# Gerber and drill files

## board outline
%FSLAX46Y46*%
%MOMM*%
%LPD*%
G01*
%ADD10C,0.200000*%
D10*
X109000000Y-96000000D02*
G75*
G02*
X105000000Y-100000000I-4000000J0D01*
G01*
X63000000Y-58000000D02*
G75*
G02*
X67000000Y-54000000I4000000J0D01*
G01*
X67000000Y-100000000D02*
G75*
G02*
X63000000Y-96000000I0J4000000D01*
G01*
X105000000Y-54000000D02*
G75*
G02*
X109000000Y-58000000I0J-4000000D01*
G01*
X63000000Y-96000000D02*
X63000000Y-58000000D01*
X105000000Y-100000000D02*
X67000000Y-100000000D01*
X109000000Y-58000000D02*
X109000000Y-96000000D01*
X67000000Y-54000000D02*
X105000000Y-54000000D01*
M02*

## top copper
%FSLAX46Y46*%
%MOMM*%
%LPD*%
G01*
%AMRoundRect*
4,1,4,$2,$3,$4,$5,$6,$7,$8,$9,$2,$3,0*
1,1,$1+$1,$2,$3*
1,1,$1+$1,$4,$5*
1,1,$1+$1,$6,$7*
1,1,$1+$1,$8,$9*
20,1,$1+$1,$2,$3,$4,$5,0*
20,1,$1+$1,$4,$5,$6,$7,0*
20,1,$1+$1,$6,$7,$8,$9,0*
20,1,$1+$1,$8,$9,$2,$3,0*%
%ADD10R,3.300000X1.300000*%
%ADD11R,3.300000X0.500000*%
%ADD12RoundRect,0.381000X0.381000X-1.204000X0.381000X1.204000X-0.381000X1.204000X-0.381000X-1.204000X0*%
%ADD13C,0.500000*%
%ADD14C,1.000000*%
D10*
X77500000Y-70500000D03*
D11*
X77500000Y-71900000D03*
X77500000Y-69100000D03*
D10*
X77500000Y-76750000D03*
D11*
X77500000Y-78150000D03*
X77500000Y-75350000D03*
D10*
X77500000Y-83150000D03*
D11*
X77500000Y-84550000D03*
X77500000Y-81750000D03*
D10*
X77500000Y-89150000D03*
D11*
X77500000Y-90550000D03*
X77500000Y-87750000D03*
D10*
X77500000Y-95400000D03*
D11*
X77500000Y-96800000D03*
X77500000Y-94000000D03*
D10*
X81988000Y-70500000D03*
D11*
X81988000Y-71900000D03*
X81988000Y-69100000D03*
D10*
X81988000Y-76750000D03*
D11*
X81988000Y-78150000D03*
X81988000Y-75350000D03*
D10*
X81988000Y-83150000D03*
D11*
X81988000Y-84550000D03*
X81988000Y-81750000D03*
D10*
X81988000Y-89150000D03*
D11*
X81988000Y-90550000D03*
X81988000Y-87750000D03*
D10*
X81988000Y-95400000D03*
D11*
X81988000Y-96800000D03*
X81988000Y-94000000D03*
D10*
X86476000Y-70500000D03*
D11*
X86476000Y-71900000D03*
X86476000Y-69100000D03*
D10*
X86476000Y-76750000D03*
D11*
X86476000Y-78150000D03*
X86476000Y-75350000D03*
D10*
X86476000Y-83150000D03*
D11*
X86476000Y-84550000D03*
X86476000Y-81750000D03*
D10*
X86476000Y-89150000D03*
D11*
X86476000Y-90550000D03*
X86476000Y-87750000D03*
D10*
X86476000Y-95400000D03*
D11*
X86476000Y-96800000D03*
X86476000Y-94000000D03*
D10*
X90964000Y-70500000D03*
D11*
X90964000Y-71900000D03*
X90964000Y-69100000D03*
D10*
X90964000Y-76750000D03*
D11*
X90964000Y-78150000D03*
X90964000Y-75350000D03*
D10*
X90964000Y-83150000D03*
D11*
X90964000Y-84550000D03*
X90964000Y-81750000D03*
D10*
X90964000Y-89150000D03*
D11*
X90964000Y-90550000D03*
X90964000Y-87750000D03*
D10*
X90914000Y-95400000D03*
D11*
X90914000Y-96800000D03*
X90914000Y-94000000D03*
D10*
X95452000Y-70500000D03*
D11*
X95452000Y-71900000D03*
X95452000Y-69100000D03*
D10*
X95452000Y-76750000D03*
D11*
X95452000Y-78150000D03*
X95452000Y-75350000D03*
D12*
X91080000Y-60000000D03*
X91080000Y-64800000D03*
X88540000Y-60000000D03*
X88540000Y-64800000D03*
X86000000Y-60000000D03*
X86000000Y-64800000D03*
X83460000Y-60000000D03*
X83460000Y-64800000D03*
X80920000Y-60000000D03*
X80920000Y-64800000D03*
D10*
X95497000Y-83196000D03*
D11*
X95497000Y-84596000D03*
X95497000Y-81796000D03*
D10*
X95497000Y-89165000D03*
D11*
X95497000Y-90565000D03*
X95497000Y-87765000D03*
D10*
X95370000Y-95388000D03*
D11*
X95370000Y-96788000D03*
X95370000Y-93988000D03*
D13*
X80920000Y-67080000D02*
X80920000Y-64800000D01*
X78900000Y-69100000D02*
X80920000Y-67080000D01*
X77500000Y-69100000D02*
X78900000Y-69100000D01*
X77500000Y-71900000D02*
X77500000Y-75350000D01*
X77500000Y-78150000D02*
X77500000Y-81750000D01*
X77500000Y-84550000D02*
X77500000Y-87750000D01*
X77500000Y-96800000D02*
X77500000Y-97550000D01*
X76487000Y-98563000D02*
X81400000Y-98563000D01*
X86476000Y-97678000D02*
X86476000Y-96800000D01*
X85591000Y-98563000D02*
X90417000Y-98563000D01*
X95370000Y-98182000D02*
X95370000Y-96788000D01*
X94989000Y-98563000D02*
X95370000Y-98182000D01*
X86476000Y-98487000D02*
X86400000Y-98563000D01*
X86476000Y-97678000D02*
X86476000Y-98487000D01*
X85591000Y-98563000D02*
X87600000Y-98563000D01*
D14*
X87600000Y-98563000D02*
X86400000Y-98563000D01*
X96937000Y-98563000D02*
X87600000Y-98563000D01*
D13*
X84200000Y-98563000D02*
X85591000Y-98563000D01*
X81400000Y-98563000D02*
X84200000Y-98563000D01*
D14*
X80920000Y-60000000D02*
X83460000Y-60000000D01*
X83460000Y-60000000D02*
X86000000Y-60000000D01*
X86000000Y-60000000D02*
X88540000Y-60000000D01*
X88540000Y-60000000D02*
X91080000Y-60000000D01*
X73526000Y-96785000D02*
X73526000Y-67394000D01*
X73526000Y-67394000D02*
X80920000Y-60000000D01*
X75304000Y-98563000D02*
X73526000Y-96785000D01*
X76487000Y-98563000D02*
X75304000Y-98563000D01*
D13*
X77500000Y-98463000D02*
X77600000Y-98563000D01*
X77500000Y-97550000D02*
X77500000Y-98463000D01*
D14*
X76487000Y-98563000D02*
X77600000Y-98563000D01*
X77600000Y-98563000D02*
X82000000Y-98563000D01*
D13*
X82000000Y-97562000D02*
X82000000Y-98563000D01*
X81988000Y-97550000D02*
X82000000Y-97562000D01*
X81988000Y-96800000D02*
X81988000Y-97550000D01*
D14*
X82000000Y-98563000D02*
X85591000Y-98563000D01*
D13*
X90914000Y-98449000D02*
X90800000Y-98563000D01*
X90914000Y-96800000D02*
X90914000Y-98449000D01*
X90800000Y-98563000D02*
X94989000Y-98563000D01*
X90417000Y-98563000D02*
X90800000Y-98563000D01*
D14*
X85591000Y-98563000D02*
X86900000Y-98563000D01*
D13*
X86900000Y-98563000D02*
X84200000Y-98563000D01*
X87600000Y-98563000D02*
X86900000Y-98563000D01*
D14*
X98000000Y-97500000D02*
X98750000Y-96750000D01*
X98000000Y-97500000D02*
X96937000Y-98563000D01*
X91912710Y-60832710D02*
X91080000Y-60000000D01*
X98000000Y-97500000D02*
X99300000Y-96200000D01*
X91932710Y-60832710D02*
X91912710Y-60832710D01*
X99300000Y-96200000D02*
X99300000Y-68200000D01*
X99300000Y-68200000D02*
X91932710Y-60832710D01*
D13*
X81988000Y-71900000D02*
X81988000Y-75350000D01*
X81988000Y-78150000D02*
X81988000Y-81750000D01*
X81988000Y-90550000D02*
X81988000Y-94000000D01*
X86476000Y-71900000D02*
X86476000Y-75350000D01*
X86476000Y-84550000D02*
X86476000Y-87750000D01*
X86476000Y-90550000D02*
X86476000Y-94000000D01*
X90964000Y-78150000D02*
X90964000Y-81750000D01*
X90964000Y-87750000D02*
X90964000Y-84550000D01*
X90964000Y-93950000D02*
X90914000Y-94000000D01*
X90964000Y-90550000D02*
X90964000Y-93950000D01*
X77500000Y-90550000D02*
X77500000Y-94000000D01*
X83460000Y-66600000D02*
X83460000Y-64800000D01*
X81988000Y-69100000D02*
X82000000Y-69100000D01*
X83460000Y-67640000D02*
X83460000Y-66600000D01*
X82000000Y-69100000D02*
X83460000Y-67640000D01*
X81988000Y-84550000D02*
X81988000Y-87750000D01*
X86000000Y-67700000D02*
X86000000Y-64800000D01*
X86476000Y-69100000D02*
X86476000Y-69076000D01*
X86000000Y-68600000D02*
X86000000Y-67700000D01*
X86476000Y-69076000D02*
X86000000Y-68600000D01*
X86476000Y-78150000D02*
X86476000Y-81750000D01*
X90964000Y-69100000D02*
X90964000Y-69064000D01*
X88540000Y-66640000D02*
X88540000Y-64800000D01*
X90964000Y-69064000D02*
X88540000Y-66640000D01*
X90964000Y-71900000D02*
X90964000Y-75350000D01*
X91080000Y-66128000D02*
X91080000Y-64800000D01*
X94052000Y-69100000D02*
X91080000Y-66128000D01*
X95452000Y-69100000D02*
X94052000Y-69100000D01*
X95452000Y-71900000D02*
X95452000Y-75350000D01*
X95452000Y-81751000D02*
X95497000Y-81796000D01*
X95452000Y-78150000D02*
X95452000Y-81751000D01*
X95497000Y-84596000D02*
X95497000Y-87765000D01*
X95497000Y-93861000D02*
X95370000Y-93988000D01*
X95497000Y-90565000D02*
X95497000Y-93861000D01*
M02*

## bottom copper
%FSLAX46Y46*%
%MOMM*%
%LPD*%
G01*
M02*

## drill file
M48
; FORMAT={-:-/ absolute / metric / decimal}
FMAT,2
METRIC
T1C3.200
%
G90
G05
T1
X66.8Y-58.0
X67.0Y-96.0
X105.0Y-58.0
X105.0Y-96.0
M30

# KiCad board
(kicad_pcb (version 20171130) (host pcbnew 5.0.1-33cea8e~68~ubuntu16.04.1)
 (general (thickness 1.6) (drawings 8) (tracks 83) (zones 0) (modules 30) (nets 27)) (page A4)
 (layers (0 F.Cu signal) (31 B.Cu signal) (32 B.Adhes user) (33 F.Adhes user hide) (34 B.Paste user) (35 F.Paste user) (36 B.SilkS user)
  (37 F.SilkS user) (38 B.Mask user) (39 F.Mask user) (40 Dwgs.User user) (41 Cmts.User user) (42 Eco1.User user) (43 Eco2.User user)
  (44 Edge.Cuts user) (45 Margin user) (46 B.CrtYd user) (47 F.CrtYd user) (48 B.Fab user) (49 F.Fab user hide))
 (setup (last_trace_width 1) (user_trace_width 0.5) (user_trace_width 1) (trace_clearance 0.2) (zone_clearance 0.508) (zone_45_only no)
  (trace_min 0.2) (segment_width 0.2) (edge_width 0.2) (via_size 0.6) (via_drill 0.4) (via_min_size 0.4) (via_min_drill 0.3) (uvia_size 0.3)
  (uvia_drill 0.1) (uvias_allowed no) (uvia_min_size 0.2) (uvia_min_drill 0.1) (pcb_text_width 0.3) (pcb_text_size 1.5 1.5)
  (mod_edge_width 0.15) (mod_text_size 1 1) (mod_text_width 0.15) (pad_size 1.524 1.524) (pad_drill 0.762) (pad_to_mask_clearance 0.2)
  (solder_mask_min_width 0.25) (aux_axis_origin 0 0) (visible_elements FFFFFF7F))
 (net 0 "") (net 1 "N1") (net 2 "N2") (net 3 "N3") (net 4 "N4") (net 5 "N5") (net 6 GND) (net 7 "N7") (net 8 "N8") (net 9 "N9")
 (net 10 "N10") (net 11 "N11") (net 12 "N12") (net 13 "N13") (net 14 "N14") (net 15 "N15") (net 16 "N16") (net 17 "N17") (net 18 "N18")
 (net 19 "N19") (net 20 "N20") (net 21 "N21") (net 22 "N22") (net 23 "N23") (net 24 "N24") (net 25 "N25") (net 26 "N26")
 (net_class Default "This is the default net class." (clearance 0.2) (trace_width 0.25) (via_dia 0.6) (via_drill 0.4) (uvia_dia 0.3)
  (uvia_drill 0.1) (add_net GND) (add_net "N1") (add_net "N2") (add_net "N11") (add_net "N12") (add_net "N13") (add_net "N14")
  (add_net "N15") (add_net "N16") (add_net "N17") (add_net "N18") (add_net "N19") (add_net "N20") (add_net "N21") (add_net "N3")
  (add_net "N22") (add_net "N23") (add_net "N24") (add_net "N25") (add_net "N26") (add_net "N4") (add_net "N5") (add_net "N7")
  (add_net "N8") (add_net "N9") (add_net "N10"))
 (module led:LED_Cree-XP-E (layer F.Cu) (at 77.5 70.5 90)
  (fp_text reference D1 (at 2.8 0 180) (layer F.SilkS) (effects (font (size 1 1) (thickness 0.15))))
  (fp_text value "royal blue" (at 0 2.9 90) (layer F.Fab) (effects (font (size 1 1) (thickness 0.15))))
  (pad 3 smd rect (at 0 -1 90) (size 1.01 0.75) (layers F.Paste))
  (pad 3 smd rect (at 0 1 90) (size 1.01 0.75) (layers F.Paste))
  (pad 3 smd rect (at 0 0 90) (size 1.01 0.75) (layers F.Paste))
  (pad 3 smd rect (at 0 0 90) (size 1.3 3.3) (layers F.Cu F.Mask))
  (pad 1 smd rect (at -1.4 0 90) (size 0.5 3.3) (layers F.Cu F.Paste F.Mask) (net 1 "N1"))
  (pad 2 smd rect (at 1.4 0 90) (size 0.5 3.3) (layers F.Cu F.Paste F.Mask) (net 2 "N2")))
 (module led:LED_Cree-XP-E (layer F.Cu) (at 77.5 76.75 90)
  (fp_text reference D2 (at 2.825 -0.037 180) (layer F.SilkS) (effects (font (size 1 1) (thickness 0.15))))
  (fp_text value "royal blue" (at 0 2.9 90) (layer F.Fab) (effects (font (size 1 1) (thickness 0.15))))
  (pad 3 smd rect (at 0 -1 90) (size 1.01 0.75) (layers F.Paste))
  (pad 3 smd rect (at 0 1 90) (size 1.01 0.75) (layers F.Paste))
  (pad 3 smd rect (at 0 0 90) (size 1.01 0.75) (layers F.Paste))
  (pad 3 smd rect (at 0 0 90) (size 1.3 3.3) (layers F.Cu F.Mask))
  (pad 1 smd rect (at -1.4 0 90) (size 0.5 3.3) (layers F.Cu F.Paste F.Mask) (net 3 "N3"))
  (pad 2 smd rect (at 1.4 0 90) (size 0.5 3.3) (layers F.Cu F.Paste F.Mask) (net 1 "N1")))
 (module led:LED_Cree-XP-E (layer F.Cu) (at 77.5 83.15 90)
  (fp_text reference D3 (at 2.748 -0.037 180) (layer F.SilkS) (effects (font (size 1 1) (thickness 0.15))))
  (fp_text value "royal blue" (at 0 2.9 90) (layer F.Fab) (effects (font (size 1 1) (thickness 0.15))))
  (pad 3 smd rect (at 0 -1 90) (size 1.01 0.75) (layers F.Paste))
  (pad 3 smd rect (at 0 1 90) (size 1.01 0.75) (layers F.Paste))
  (pad 3 smd rect (at 0 0 90) (size 1.01 0.75) (layers F.Paste))
  (pad 3 smd rect (at 0 0 90) (size 1.3 3.3) (layers F.Cu F.Mask))
  (pad 1 smd rect (at -1.4 0 90) (size 0.5 3.3) (layers F.Cu F.Paste F.Mask) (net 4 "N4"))
  (pad 2 smd rect (at 1.4 0 90) (size 0.5 3.3) (layers F.Cu F.Paste F.Mask) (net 3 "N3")))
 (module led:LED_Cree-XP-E (layer F.Cu) (at 77.5 89.15 90)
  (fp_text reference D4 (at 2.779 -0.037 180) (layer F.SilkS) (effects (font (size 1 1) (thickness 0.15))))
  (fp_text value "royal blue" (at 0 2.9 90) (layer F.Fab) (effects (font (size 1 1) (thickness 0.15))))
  (pad 3 smd rect (at 0 -1 90) (size 1.01 0.75) (layers F.Paste))
  (pad 3 smd rect (at 0 1 90) (size 1.01 0.75) (layers F.Paste))
  (pad 3 smd rect (at 0 0 90) (size 1.01 0.75) (layers F.Paste))
  (pad 3 smd rect (at 0 0 90) (size 1.3 3.3) (layers F.Cu F.Mask))
  (pad 1 smd rect (at -1.4 0 90) (size 0.5 3.3) (layers F.Cu F.Paste F.Mask) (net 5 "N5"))
  (pad 2 smd rect (at 1.4 0 90) (size 0.5 3.3) (layers F.Cu F.Paste F.Mask) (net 4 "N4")))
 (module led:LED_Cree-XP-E (layer F.Cu) (at 77.5 95.4 90)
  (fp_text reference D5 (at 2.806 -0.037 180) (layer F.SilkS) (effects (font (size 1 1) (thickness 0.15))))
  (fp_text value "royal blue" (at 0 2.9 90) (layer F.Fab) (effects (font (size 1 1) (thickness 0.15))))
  (pad 3 smd rect (at 0 -1 90) (size 1.01 0.75) (layers F.Paste))
  (pad 3 smd rect (at 0 1 90) (size 1.01 0.75) (layers F.Paste))
  (pad 3 smd rect (at 0 0 90) (size 1.01 0.75) (layers F.Paste))
  (pad 3 smd rect (at 0 0 90) (size 1.3 3.3) (layers F.Cu F.Mask))
  (pad 1 smd rect (at -1.4 0 90) (size 0.5 3.3) (layers F.Cu F.Paste F.Mask) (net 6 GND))
  (pad 2 smd rect (at 1.4 0 90) (size 0.5 3.3) (layers F.Cu F.Paste F.Mask) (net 5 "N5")))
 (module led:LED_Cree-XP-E (layer F.Cu) (at 81.988 70.5 90)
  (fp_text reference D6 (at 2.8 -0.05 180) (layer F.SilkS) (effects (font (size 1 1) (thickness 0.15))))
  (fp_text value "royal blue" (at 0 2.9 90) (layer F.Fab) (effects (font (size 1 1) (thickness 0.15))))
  (pad 3 smd rect (at 0 -1 90) (size 1.01 0.75) (layers F.Paste))
  (pad 3 smd rect (at 0 1 90) (size 1.01 0.75) (layers F.Paste))
  (pad 3 smd rect (at 0 0 90) (size 1.01 0.75) (layers F.Paste))
  (pad 3 smd rect (at 0 0 90) (size 1.3 3.3) (layers F.Cu F.Mask))
  (pad 1 smd rect (at -1.4 0 90) (size 0.5 3.3) (layers F.Cu F.Paste F.Mask) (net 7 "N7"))
  (pad 2 smd rect (at 1.4 0 90) (size 0.5 3.3) (layers F.Cu F.Paste F.Mask) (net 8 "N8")))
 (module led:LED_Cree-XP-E (layer F.Cu) (at 81.988 76.75 90)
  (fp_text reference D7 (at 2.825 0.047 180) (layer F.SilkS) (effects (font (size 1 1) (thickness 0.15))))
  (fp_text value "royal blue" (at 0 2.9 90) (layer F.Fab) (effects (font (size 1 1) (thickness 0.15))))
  (pad 3 smd rect (at 0 -1 90) (size 1.01 0.75) (layers F.Paste))
  (pad 3 smd rect (at 0 1 90) (size 1.01 0.75) (layers F.Paste))
  (pad 3 smd rect (at 0 0 90) (size 1.01 0.75) (layers F.Paste))
  (pad 3 smd rect (at 0 0 90) (size 1.3 3.3) (layers F.Cu F.Mask))
  (pad 1 smd rect (at -1.4 0 90) (size 0.5 3.3) (layers F.Cu F.Paste F.Mask) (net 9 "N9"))
  (pad 2 smd rect (at 1.4 0 90) (size 0.5 3.3) (layers F.Cu F.Paste F.Mask) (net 7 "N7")))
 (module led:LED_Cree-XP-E (layer F.Cu) (at 81.988 83.15 90)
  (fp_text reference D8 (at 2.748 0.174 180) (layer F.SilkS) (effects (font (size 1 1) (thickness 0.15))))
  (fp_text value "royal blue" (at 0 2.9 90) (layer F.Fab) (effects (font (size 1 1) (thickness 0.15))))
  (pad 3 smd rect (at 0 -1 90) (size 1.01 0.75) (layers F.Paste))
  (pad 3 smd rect (at 0 1 90) (size 1.01 0.75) (layers F.Paste))
  (pad 3 smd rect (at 0 0 90) (size 1.01 0.75) (layers F.Paste))
  (pad 3 smd rect (at 0 0 90) (size 1.3 3.3) (layers F.Cu F.Mask))
  (pad 1 smd rect (at -1.4 0 90) (size 0.5 3.3) (layers F.Cu F.Paste F.Mask) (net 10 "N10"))
  (pad 2 smd rect (at 1.4 0 90) (size 0.5 3.3) (layers F.Cu F.Paste F.Mask) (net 9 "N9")))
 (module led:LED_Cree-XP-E (layer F.Cu) (at 81.988 89.15 90)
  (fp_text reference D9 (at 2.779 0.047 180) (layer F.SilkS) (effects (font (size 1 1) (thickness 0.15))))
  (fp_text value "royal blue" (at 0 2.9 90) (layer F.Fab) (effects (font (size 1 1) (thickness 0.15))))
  (pad 3 smd rect (at 0 -1 90) (size 1.01 0.75) (layers F.Paste))
  (pad 3 smd rect (at 0 1 90) (size 1.01 0.75) (layers F.Paste))
  (pad 3 smd rect (at 0 0 90) (size 1.01 0.75) (layers F.Paste))
  (pad 3 smd rect (at 0 0 90) (size 1.3 3.3) (layers F.Cu F.Mask))
  (pad 1 smd rect (at -1.4 0 90) (size 0.5 3.3) (layers F.Cu F.Paste F.Mask) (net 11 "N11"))
  (pad 2 smd rect (at 1.4 0 90) (size 0.5 3.3) (layers F.Cu F.Paste F.Mask) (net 10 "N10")))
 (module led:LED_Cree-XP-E (layer F.Cu) (at 81.988 95.4 90)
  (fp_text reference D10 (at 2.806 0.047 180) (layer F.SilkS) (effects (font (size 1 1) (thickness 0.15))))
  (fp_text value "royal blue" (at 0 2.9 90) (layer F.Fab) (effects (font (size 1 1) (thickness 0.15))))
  (pad 3 smd rect (at 0 -1 90) (size 1.01 0.75) (layers F.Paste))
  (pad 3 smd rect (at 0 1 90) (size 1.01 0.75) (layers F.Paste))
  (pad 3 smd rect (at 0 0 90) (size 1.01 0.75) (layers F.Paste))
  (pad 3 smd rect (at 0 0 90) (size 1.3 3.3) (layers F.Cu F.Mask))
  (pad 1 smd rect (at -1.4 0 90) (size 0.5 3.3) (layers F.Cu F.Paste F.Mask) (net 6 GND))
  (pad 2 smd rect (at 1.4 0 90) (size 0.5 3.3) (layers F.Cu F.Paste F.Mask) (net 11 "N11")))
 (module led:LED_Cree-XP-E (layer F.Cu) (at 86.476 70.5 90)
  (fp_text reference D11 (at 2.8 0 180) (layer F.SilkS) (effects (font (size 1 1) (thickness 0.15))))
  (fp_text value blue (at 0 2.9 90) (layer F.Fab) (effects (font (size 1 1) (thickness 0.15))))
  (pad 3 smd rect (at 0 -1 90) (size 1.01 0.75) (layers F.Paste))
  (pad 3 smd rect (at 0 1 90) (size 1.01 0.75) (layers F.Paste))
  (pad 3 smd rect (at 0 0 90) (size 1.01 0.75) (layers F.Paste))
  (pad 3 smd rect (at 0 0 90) (size 1.3 3.3) (layers F.Cu F.Mask))
  (pad 1 smd rect (at -1.4 0 90) (size 0.5 3.3) (layers F.Cu F.Paste F.Mask) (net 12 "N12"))
  (pad 2 smd rect (at 1.4 0 90) (size 0.5 3.3) (layers F.Cu F.Paste F.Mask) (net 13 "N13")))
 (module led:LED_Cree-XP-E (layer F.Cu) (at 86.476 76.75 90)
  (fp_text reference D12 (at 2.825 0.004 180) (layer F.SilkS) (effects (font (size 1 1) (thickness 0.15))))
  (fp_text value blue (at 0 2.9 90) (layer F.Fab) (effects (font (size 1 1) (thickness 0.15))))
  (pad 3 smd rect (at 0 -1 90) (size 1.01 0.75) (layers F.Paste))
  (pad 3 smd rect (at 0 1 90) (size 1.01 0.75) (layers F.Paste))
  (pad 3 smd rect (at 0 0 90) (size 1.01 0.75) (layers F.Paste))
  (pad 3 smd rect (at 0 0 90) (size 1.3 3.3) (layers F.Cu F.Mask))
  (pad 1 smd rect (at -1.4 0 90) (size 0.5 3.3) (layers F.Cu F.Paste F.Mask) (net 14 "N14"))
  (pad 2 smd rect (at 1.4 0 90) (size 0.5 3.3) (layers F.Cu F.Paste F.Mask) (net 12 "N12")))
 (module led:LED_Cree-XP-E (layer F.Cu) (at 86.476 83.15 90)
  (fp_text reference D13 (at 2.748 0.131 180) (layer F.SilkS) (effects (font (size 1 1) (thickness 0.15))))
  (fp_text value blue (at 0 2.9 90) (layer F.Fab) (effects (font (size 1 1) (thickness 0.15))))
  (pad 3 smd rect (at 0 -1 90) (size 1.01 0.75) (layers F.Paste))
  (pad 3 smd rect (at 0 1 90) (size 1.01 0.75) (layers F.Paste))
  (pad 3 smd rect (at 0 0 90) (size 1.01 0.75) (layers F.Paste))
  (pad 3 smd rect (at 0 0 90) (size 1.3 3.3) (layers F.Cu F.Mask))
  (pad 1 smd rect (at -1.4 0 90) (size 0.5 3.3) (layers F.Cu F.Paste F.Mask) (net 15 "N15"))
  (pad 2 smd rect (at 1.4 0 90) (size 0.5 3.3) (layers F.Cu F.Paste F.Mask) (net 14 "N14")))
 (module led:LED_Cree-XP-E (layer F.Cu) (at 86.476 89.15 90)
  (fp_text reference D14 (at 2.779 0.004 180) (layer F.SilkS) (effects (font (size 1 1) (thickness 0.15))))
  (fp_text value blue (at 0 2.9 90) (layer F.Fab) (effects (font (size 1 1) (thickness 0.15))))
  (pad 3 smd rect (at 0 -1 90) (size 1.01 0.75) (layers F.Paste))
  (pad 3 smd rect (at 0 1 90) (size 1.01 0.75) (layers F.Paste))
  (pad 3 smd rect (at 0 0 90) (size 1.01 0.75) (layers F.Paste))
  (pad 3 smd rect (at 0 0 90) (size 1.3 3.3) (layers F.Cu F.Mask))
  (pad 1 smd rect (at -1.4 0 90) (size 0.5 3.3) (layers F.Cu F.Paste F.Mask) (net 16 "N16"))
  (pad 2 smd rect (at 1.4 0 90) (size 0.5 3.3) (layers F.Cu F.Paste F.Mask) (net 15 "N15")))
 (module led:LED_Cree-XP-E (layer F.Cu) (at 86.476 95.4 90)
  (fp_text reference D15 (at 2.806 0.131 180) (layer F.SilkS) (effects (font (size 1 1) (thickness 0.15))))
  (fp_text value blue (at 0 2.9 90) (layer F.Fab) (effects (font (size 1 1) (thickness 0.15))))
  (pad 3 smd rect (at 0 -1 90) (size 1.01 0.75) (layers F.Paste))
  (pad 3 smd rect (at 0 1 90) (size 1.01 0.75) (layers F.Paste))
  (pad 3 smd rect (at 0 0 90) (size 1.01 0.75) (layers F.Paste))
  (pad 3 smd rect (at 0 0 90) (size 1.3 3.3) (layers F.Cu F.Mask))
  (pad 1 smd rect (at -1.4 0 90) (size 0.5 3.3) (layers F.Cu F.Paste F.Mask) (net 6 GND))
  (pad 2 smd rect (at 1.4 0 90) (size 0.5 3.3) (layers F.Cu F.Paste F.Mask) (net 16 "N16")))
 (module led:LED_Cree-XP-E (layer F.Cu) (at 90.964 70.5 90)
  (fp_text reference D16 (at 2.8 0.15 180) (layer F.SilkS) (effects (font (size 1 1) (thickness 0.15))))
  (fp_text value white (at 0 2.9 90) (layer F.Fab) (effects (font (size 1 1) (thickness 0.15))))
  (pad 3 smd rect (at 0 -1 90) (size 1.01 0.75) (layers F.Paste))
  (pad 3 smd rect (at 0 1 90) (size 1.01 0.75) (layers F.Paste))
  (pad 3 smd rect (at 0 0 90) (size 1.01 0.75) (layers F.Paste))
  (pad 3 smd rect (at 0 0 90) (size 1.3 3.3) (layers F.Cu F.Mask))
  (pad 1 smd rect (at -1.4 0 90) (size 0.5 3.3) (layers F.Cu F.Paste F.Mask) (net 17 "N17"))
  (pad 2 smd rect (at 1.4 0 90) (size 0.5 3.3) (layers F.Cu F.Paste F.Mask) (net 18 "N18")))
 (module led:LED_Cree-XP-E (layer F.Cu) (at 90.964 76.75 90)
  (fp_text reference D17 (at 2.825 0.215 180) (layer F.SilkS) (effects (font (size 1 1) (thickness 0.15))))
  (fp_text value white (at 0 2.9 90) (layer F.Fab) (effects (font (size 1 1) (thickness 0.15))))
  (pad 3 smd rect (at 0 -1 90) (size 1.01 0.75) (layers F.Paste))
  (pad 3 smd rect (at 0 1 90) (size 1.01 0.75) (layers F.Paste))
  (pad 3 smd rect (at 0 0 90) (size 1.01 0.75) (layers F.Paste))
  (pad 3 smd rect (at 0 0 90) (size 1.3 3.3) (layers F.Cu F.Mask))
  (pad 1 smd rect (at -1.4 0 90) (size 0.5 3.3) (layers F.Cu F.Paste F.Mask) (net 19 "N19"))
  (pad 2 smd rect (at 1.4 0 90) (size 0.5 3.3) (layers F.Cu F.Paste F.Mask) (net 17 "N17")))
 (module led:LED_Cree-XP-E (layer F.Cu) (at 90.964 83.15 90)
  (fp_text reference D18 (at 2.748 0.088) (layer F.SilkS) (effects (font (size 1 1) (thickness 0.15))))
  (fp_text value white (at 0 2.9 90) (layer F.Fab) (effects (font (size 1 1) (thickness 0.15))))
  (pad 3 smd rect (at 0 -1 90) (size 1.01 0.75) (layers F.Paste))
  (pad 3 smd rect (at 0 1 90) (size 1.01 0.75) (layers F.Paste))
  (pad 3 smd rect (at 0 0 90) (size 1.01 0.75) (layers F.Paste))
  (pad 3 smd rect (at 0 0 90) (size 1.3 3.3) (layers F.Cu F.Mask))
  (pad 1 smd rect (at -1.4 0 90) (size 0.5 3.3) (layers F.Cu F.Paste F.Mask) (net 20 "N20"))
  (pad 2 smd rect (at 1.4 0 90) (size 0.5 3.3) (layers F.Cu F.Paste F.Mask) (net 19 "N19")))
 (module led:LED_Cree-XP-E (layer F.Cu) (at 90.964 89.15 90)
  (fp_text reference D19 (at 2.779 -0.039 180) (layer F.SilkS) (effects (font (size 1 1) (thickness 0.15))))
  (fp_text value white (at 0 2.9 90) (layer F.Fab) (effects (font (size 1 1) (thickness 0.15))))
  (pad 3 smd rect (at 0 -1 90) (size 1.01 0.75) (layers F.Paste))
  (pad 3 smd rect (at 0 1 90) (size 1.01 0.75) (layers F.Paste))
  (pad 3 smd rect (at 0 0 90) (size 1.01 0.75) (layers F.Paste))
  (pad 3 smd rect (at 0 0 90) (size 1.3 3.3) (layers F.Cu F.Mask))
  (pad 1 smd rect (at -1.4 0 90) (size 0.5 3.3) (layers F.Cu F.Paste F.Mask) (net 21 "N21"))
  (pad 2 smd rect (at 1.4 0 90) (size 0.5 3.3) (layers F.Cu F.Paste F.Mask) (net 20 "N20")))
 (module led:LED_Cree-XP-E (layer F.Cu) (at 90.914 95.4 90)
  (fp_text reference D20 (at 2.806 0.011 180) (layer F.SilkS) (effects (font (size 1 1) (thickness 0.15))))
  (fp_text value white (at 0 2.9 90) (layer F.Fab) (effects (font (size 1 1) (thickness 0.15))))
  (pad 3 smd rect (at 0 -1 90) (size 1.01 0.75) (layers F.Paste))
  (pad 3 smd rect (at 0 1 90) (size 1.01 0.75) (layers F.Paste))
  (pad 3 smd rect (at 0 0 90) (size 1.01 0.75) (layers F.Paste))
  (pad 3 smd rect (at 0 0 90) (size 1.3 3.3) (layers F.Cu F.Mask))
  (pad 1 smd rect (at -1.4 0 90) (size 0.5 3.3) (layers F.Cu F.Paste F.Mask) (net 6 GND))
  (pad 2 smd rect (at 1.4 0 90) (size 0.5 3.3) (layers F.Cu F.Paste F.Mask) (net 21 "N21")))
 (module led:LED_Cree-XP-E (layer F.Cu) (at 95.452 70.5 90)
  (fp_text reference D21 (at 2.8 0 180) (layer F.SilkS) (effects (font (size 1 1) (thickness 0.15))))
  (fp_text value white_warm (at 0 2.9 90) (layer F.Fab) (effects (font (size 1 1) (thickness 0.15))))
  (pad 3 smd rect (at 0 -1 90) (size 1.01 0.75) (layers F.Paste))
  (pad 3 smd rect (at 0 1 90) (size 1.01 0.75) (layers F.Paste))
  (pad 3 smd rect (at 0 0 90) (size 1.01 0.75) (layers F.Paste))
  (pad 3 smd rect (at 0 0 90) (size 1.3 3.3) (layers F.Cu F.Mask))
  (pad 1 smd rect (at -1.4 0 90) (size 0.5 3.3) (layers F.Cu F.Paste F.Mask) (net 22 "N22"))
  (pad 2 smd rect (at 1.4 0 90) (size 0.5 3.3) (layers F.Cu F.Paste F.Mask) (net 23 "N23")))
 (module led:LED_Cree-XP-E (layer F.Cu) (at 95.452 76.75 90)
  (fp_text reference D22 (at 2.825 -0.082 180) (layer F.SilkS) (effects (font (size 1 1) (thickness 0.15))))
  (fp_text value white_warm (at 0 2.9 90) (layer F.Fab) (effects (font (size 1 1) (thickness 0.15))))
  (pad 3 smd rect (at 0 -1 90) (size 1.01 0.75) (layers F.Paste))
  (pad 3 smd rect (at 0 1 90) (size 1.01 0.75) (layers F.Paste))
  (pad 3 smd rect (at 0 0 90) (size 1.01 0.75) (layers F.Paste))
  (pad 3 smd rect (at 0 0 90) (size 1.3 3.3) (layers F.Cu F.Mask))
  (pad 1 smd rect (at -1.4 0 90) (size 0.5 3.3) (layers F.Cu F.Paste F.Mask) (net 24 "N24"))
  (pad 2 smd rect (at 1.4 0 90) (size 0.5 3.3) (layers F.Cu F.Paste F.Mask) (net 22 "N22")))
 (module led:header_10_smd (layer F.Cu) (at 80.92 64.8 90)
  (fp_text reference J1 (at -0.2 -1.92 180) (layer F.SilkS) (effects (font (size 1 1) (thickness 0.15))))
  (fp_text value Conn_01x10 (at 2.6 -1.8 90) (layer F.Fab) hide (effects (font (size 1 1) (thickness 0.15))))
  (pad 1 smd roundrect (at 4.8 10.16 90) (size 3.17 1.524) (layers F.Cu F.Paste F.Mask) (roundrect_rratio 0.25) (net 6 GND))
  (pad 2 smd roundrect (at 0 10.16 90) (size 3.17 1.524) (layers F.Cu F.Paste F.Mask) (roundrect_rratio 0.25) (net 23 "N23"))
  (pad 3 smd roundrect (at 4.8 7.62 90) (size 3.17 1.524) (layers F.Cu F.Paste F.Mask) (roundrect_rratio 0.25) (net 6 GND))
  (pad 4 smd roundrect (at 0 7.62 90) (size 3.17 1.524) (layers F.Cu F.Paste F.Mask) (roundrect_rratio 0.25) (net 18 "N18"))
  (pad 5 smd roundrect (at 4.8 5.08 90) (size 3.17 1.524) (layers F.Cu F.Paste F.Mask) (roundrect_rratio 0.25) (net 6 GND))
  (pad 6 smd roundrect (at 0 5.08 90) (size 3.17 1.524) (layers F.Cu F.Paste F.Mask) (roundrect_rratio 0.25) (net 13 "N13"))
  (pad 7 smd roundrect (at 4.8 2.54 90) (size 3.17 1.524) (layers F.Cu F.Paste F.Mask) (roundrect_rratio 0.25) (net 6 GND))
  (pad 8 smd roundrect (at 0 2.54 90) (size 3.17 1.524) (layers F.Cu F.Paste F.Mask) (roundrect_rratio 0.25) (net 8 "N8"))
  (pad 9 smd roundrect (at 4.8 0 90) (size 3.17 1.524) (layers F.Cu F.Paste F.Mask) (roundrect_rratio 0.25) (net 6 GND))
  (pad 10 smd roundrect (at 0 0 90) (size 3.17 1.524) (layers F.Cu F.Paste F.Mask) (roundrect_rratio 0.25) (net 2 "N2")))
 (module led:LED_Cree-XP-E (layer F.Cu) (at 95.497 83.196 90)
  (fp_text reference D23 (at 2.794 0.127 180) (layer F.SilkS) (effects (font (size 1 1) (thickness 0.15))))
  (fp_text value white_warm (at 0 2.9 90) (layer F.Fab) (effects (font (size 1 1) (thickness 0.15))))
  (pad 3 smd rect (at 0 -1 90) (size 1.01 0.75) (layers F.Paste))
  (pad 3 smd rect (at 0 1 90) (size 1.01 0.75) (layers F.Paste))
  (pad 3 smd rect (at 0 0 90) (size 1.01 0.75) (layers F.Paste))
  (pad 3 smd rect (at 0 0 90) (size 1.3 3.3) (layers F.Cu F.Mask))
  (pad 1 smd rect (at -1.4 0 90) (size 0.5 3.3) (layers F.Cu F.Paste F.Mask) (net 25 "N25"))
  (pad 2 smd rect (at 1.4 0 90) (size 0.5 3.3) (layers F.Cu F.Paste F.Mask) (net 24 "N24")))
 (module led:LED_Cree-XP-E (layer F.Cu) (at 95.497 89.165 90)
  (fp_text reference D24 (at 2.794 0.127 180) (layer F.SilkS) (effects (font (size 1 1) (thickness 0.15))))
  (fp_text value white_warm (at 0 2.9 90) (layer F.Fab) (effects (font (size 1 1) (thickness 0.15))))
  (pad 3 smd rect (at 0 -1 90) (size 1.01 0.75) (layers F.Paste))
  (pad 3 smd rect (at 0 1 90) (size 1.01 0.75) (layers F.Paste))
  (pad 3 smd rect (at 0 0 90) (size 1.01 0.75) (layers F.Paste))
  (pad 3 smd rect (at 0 0 90) (size 1.3 3.3) (layers F.Cu F.Mask))
  (pad 1 smd rect (at -1.4 0 90) (size 0.5 3.3) (layers F.Cu F.Paste F.Mask) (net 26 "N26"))
  (pad 2 smd rect (at 1.4 0 90) (size 0.5 3.3) (layers F.Cu F.Paste F.Mask) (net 25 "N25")))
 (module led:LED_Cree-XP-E (layer F.Cu) (at 95.37 95.388 90)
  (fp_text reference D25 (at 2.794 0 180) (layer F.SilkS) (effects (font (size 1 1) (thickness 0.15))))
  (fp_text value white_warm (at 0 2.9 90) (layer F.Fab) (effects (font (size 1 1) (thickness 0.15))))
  (pad 3 smd rect (at 0 -1 90) (size 1.01 0.75) (layers F.Paste))
  (pad 3 smd rect (at 0 1 90) (size 1.01 0.75) (layers F.Paste))
  (pad 3 smd rect (at 0 0 90) (size 1.01 0.75) (layers F.Paste))
  (pad 3 smd rect (at 0 0 90) (size 1.3 3.3) (layers F.Cu F.Mask))
  (pad 1 smd rect (at -1.4 0 90) (size 0.5 3.3) (layers F.Cu F.Paste F.Mask) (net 6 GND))
  (pad 2 smd rect (at 1.4 0 90) (size 0.5 3.3) (layers F.Cu F.Paste F.Mask) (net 26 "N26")))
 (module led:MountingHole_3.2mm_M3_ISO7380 (layer F.Cu) (at 66.8 58)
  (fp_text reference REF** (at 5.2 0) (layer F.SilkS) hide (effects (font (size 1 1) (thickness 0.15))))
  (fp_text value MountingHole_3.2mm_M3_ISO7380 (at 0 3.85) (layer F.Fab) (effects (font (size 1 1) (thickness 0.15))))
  (pad 1 np_thru_hole circle (at 0 0) (size 3.2 3.2) (drill 3.2) (layers *.Cu *.Mask)))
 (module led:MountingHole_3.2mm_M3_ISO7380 (layer F.Cu) (at 105 58)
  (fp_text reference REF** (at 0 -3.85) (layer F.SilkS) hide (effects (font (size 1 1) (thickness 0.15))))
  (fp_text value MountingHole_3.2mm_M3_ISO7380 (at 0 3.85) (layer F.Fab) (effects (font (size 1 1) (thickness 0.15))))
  (pad 1 np_thru_hole circle (at 0 0) (size 3.2 3.2) (drill 3.2) (layers *.Cu *.Mask)))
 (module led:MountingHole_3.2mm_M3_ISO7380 (layer F.Cu) (at 67 96)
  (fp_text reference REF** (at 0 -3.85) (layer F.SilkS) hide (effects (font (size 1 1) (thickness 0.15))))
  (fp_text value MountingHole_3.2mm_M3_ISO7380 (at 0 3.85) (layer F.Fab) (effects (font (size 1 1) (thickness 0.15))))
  (pad 1 np_thru_hole circle (at 0 0) (size 3.2 3.2) (drill 3.2) (layers *.Cu *.Mask)))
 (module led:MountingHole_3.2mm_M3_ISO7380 (layer F.Cu) (at 105 96)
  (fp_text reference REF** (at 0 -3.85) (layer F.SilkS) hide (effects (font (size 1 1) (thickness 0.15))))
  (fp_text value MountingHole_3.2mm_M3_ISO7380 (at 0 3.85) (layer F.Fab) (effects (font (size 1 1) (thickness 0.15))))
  (pad 1 np_thru_hole circle (at 0 0) (size 3.2 3.2) (drill 3.2) (layers *.Cu *.Mask)))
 (gr_arc (start 105 96) (end 105 100) (angle -90) (layer Edge.Cuts) (width 0.2))
 (gr_arc (start 67 58) (end 67 54) (angle -90) (layer Edge.Cuts) (width 0.2))
 (gr_arc (start 67 96) (end 63 96) (angle -90) (layer Edge.Cuts) (width 0.2))
 (gr_arc (start 105 58) (end 109 58) (angle -90) (layer Edge.Cuts) (width 0.2))
 (gr_line (start 63 96) (end 63 58) (angle 90) (layer Edge.Cuts) (width 0.2))
 (gr_line (start 105 100) (end 67 100) (angle 90) (layer Edge.Cuts) (width 0.2))
 (gr_line (start 109 58) (end 109 96) (angle 90) (layer Edge.Cuts) (width 0.2))
 (gr_line (start 67 54) (end 105 54) (angle 90) (layer Edge.Cuts) (width 0.2))
 (segment (start 80.92 67.08) (end 80.92 64.8) (width 0.5) (layer F.Cu) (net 2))
 (segment (start 78.9 69.1) (end 80.92 67.08) (width 0.5) (layer F.Cu) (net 2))
 (segment (start 77.5 69.1) (end 78.9 69.1) (width 0.5) (layer F.Cu) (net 2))
 (segment (start 77.5 71.9) (end 77.5 75.35) (width 0.5) (layer F.Cu) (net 1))
 (segment (start 77.5 78.15) (end 77.5 81.75) (width 0.5) (layer F.Cu) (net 3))
 (segment (start 77.5 84.55) (end 77.5 87.75) (width 0.5) (layer F.Cu) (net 4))
 (segment (start 77.5 96.8) (end 77.5 97.55) (width 0.5) (layer F.Cu) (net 6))
 (segment (start 76.487 98.563) (end 81.4 98.563) (width 0.5) (layer F.Cu) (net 6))
 (segment (start 86.476 97.678) (end 86.476 96.8) (width 0.5) (layer F.Cu) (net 6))
 (segment (start 85.591 98.563) (end 90.417 98.563) (width 0.5) (layer F.Cu) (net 6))
 (segment (start 95.37 98.182) (end 95.37 96.788) (width 0.5) (layer F.Cu) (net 6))
 (segment (start 94.989 98.563) (end 95.37 98.182) (width 0.5) (layer F.Cu) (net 6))
 (segment (start 86.476 98.487) (end 86.4 98.563) (width 0.5) (layer F.Cu) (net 6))
 (segment (start 86.476 97.678) (end 86.476 98.487) (width 0.5) (layer F.Cu) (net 6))
 (segment (start 85.591 98.563) (end 87.6 98.563) (width 0.5) (layer F.Cu) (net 6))
 (segment (start 87.6 98.563) (end 86.4 98.563) (width 1) (layer F.Cu) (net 6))
 (segment (start 96.937 98.563) (end 87.6 98.563) (width 1) (layer F.Cu) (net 6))
 (segment (start 84.2 98.563) (end 85.591 98.563) (width 0.5) (layer F.Cu) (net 6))
 (segment (start 81.4 98.563) (end 84.2 98.563) (width 0.5) (layer F.Cu) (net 6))
 (segment (start 80.92 60) (end 83.46 60) (width 1) (layer F.Cu) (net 6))
 (segment (start 83.46 60) (end 86 60) (width 1) (layer F.Cu) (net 6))
 (segment (start 86 60) (end 88.54 60) (width 1) (layer F.Cu) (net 6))
 (segment (start 88.54 60) (end 91.08 60) (width 1) (layer F.Cu) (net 6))
 (segment (start 73.526 96.785) (end 73.526 67.394) (width 1) (layer F.Cu) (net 6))
 (segment (start 73.526 67.394) (end 80.92 60) (width 1) (layer F.Cu) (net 6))
 (segment (start 75.304 98.563) (end 73.526 96.785) (width 1) (layer F.Cu) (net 6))
 (segment (start 76.487 98.563) (end 75.304 98.563) (width 1) (layer F.Cu) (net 6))
 (segment (start 77.5 98.463) (end 77.6 98.563) (width 0.5) (layer F.Cu) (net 6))
 (segment (start 77.5 97.55) (end 77.5 98.463) (width 0.5) (layer F.Cu) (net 6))
 (segment (start 76.487 98.563) (end 77.6 98.563) (width 1) (layer F.Cu) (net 6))
 (segment (start 77.6 98.563) (end 82 98.563) (width 1) (layer F.Cu) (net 6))
 (segment (start 82 97.562) (end 82 98.563) (width 0.5) (layer F.Cu) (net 6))
 (segment (start 81.988 97.55) (end 82 97.562) (width 0.5) (layer F.Cu) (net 6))
 (segment (start 81.988 96.8) (end 81.988 97.55) (width 0.5) (layer F.Cu) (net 6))
 (segment (start 82 98.563) (end 85.591 98.563) (width 1) (layer F.Cu) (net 6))
 (segment (start 90.914 98.449) (end 90.8 98.563) (width 0.5) (layer F.Cu) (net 6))
 (segment (start 90.914 96.8) (end 90.914 98.449) (width 0.5) (layer F.Cu) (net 6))
 (segment (start 90.8 98.563) (end 94.989 98.563) (width 0.5) (layer F.Cu) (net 6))
 (segment (start 90.417 98.563) (end 90.8 98.563) (width 0.5) (layer F.Cu) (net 6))
 (segment (start 85.591 98.563) (end 86.9 98.563) (width 1) (layer F.Cu) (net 6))
 (segment (start 86.9 98.563) (end 84.2 98.563) (width 0.5) (layer F.Cu) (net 6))
 (segment (start 87.6 98.563) (end 86.9 98.563) (width 0.5) (layer F.Cu) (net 6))
 (segment (start 98 97.5) (end 98.75 96.75) (width 1) (layer F.Cu) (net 6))
 (segment (start 98 97.5) (end 96.937 98.563) (width 1) (layer F.Cu) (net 6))
 (segment (start 91.91271 60.83271) (end 91.08 60) (width 1) (layer F.Cu) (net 6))
 (segment (start 98 97.5) (end 99.3 96.2) (width 1) (layer F.Cu) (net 6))
 (segment (start 91.93271 60.83271) (end 91.91271 60.83271) (width 1) (layer F.Cu) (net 6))
 (segment (start 99.3 96.2) (end 99.3 68.2) (width 1) (layer F.Cu) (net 6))
 (segment (start 99.3 68.2) (end 91.93271 60.83271) (width 1) (layer F.Cu) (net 6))
 (segment (start 81.988 71.9) (end 81.988 75.35) (width 0.5) (layer F.Cu) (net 7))
 (segment (start 81.988 78.15) (end 81.988 81.75) (width 0.5) (layer F.Cu) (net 9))
 (segment (start 81.988 90.55) (end 81.988 94) (width 0.5) (layer F.Cu) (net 11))
 (segment (start 86.476 71.9) (end 86.476 75.35) (width 0.5) (layer F.Cu) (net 12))
 (segment (start 86.476 84.55) (end 86.476 87.75) (width 0.5) (layer F.Cu) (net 15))
 (segment (start 86.476 90.55) (end 86.476 94) (width 0.5) (layer F.Cu) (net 16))
 (segment (start 90.964 78.15) (end 90.964 81.75) (width 0.5) (layer F.Cu) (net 19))
 (segment (start 90.964 87.75) (end 90.964 84.55) (width 0.5) (layer F.Cu) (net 20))
 (segment (start 90.964 93.95) (end 90.914 94) (width 0.5) (layer F.Cu) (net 21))
 (segment (start 90.964 90.55) (end 90.964 93.95) (width 0.5) (layer F.Cu) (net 21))
 (segment (start 77.5 90.55) (end 77.5 94) (width 0.5) (layer F.Cu) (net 5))
 (segment (start 83.46 66.6) (end 83.46 64.8) (width 0.5) (layer F.Cu) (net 8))
 (segment (start 81.988 69.1) (end 82 69.1) (width 0.5) (layer F.Cu) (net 8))
 (segment (start 83.46 67.64) (end 83.46 66.6) (width 0.5) (layer F.Cu) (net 8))
 (segment (start 82 69.1) (end 83.46 67.64) (width 0.5) (layer F.Cu) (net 8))
 (segment (start 81.988 84.55) (end 81.988 87.75) (width 0.5) (layer F.Cu) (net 10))
 (segment (start 86 67.7) (end 86 64.8) (width 0.5) (layer F.Cu) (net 13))
 (segment (start 86.476 69.1) (end 86.476 69.076) (width 0.5) (layer F.Cu) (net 13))
 (segment (start 86 68.6) (end 86 67.7) (width 0.5) (layer F.Cu) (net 13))
 (segment (start 86.476 69.076) (end 86 68.6) (width 0.5) (layer F.Cu) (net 13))
 (segment (start 86.476 78.15) (end 86.476 81.75) (width 0.5) (layer F.Cu) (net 14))
 (segment (start 90.964 69.1) (end 90.964 69.064) (width 0.5) (layer F.Cu) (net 18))
 (segment (start 88.54 66.64) (end 88.54 64.8) (width 0.5) (layer F.Cu) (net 18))
 (segment (start 90.964 69.064) (end 88.54 66.64) (width 0.5) (layer F.Cu) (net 18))
 (segment (start 90.964 71.9) (end 90.964 75.35) (width 0.5) (layer F.Cu) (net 17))
 (segment (start 91.08 66.128) (end 91.08 64.8) (width 0.5) (layer F.Cu) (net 23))
 (segment (start 94.052 69.1) (end 91.08 66.128) (width 0.5) (layer F.Cu) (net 23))
 (segment (start 95.452 69.1) (end 94.052 69.1) (width 0.5) (layer F.Cu) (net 23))
 (segment (start 95.452 71.9) (end 95.452 75.35) (width 0.5) (layer F.Cu) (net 22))
 (segment (start 95.452 81.751) (end 95.497 81.796) (width 0.5) (layer F.Cu) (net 24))
 (segment (start 95.452 78.15) (end 95.452 81.751) (width 0.5) (layer F.Cu) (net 24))
 (segment (start 95.497 84.596) (end 95.497 87.765) (width 0.5) (layer F.Cu) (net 25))
 (segment (start 95.497 93.861) (end 95.37 93.988) (width 0.5) (layer F.Cu) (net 26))
 (segment (start 95.497 90.565) (end 95.497 93.861) (width 0.5) (layer F.Cu) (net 26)))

